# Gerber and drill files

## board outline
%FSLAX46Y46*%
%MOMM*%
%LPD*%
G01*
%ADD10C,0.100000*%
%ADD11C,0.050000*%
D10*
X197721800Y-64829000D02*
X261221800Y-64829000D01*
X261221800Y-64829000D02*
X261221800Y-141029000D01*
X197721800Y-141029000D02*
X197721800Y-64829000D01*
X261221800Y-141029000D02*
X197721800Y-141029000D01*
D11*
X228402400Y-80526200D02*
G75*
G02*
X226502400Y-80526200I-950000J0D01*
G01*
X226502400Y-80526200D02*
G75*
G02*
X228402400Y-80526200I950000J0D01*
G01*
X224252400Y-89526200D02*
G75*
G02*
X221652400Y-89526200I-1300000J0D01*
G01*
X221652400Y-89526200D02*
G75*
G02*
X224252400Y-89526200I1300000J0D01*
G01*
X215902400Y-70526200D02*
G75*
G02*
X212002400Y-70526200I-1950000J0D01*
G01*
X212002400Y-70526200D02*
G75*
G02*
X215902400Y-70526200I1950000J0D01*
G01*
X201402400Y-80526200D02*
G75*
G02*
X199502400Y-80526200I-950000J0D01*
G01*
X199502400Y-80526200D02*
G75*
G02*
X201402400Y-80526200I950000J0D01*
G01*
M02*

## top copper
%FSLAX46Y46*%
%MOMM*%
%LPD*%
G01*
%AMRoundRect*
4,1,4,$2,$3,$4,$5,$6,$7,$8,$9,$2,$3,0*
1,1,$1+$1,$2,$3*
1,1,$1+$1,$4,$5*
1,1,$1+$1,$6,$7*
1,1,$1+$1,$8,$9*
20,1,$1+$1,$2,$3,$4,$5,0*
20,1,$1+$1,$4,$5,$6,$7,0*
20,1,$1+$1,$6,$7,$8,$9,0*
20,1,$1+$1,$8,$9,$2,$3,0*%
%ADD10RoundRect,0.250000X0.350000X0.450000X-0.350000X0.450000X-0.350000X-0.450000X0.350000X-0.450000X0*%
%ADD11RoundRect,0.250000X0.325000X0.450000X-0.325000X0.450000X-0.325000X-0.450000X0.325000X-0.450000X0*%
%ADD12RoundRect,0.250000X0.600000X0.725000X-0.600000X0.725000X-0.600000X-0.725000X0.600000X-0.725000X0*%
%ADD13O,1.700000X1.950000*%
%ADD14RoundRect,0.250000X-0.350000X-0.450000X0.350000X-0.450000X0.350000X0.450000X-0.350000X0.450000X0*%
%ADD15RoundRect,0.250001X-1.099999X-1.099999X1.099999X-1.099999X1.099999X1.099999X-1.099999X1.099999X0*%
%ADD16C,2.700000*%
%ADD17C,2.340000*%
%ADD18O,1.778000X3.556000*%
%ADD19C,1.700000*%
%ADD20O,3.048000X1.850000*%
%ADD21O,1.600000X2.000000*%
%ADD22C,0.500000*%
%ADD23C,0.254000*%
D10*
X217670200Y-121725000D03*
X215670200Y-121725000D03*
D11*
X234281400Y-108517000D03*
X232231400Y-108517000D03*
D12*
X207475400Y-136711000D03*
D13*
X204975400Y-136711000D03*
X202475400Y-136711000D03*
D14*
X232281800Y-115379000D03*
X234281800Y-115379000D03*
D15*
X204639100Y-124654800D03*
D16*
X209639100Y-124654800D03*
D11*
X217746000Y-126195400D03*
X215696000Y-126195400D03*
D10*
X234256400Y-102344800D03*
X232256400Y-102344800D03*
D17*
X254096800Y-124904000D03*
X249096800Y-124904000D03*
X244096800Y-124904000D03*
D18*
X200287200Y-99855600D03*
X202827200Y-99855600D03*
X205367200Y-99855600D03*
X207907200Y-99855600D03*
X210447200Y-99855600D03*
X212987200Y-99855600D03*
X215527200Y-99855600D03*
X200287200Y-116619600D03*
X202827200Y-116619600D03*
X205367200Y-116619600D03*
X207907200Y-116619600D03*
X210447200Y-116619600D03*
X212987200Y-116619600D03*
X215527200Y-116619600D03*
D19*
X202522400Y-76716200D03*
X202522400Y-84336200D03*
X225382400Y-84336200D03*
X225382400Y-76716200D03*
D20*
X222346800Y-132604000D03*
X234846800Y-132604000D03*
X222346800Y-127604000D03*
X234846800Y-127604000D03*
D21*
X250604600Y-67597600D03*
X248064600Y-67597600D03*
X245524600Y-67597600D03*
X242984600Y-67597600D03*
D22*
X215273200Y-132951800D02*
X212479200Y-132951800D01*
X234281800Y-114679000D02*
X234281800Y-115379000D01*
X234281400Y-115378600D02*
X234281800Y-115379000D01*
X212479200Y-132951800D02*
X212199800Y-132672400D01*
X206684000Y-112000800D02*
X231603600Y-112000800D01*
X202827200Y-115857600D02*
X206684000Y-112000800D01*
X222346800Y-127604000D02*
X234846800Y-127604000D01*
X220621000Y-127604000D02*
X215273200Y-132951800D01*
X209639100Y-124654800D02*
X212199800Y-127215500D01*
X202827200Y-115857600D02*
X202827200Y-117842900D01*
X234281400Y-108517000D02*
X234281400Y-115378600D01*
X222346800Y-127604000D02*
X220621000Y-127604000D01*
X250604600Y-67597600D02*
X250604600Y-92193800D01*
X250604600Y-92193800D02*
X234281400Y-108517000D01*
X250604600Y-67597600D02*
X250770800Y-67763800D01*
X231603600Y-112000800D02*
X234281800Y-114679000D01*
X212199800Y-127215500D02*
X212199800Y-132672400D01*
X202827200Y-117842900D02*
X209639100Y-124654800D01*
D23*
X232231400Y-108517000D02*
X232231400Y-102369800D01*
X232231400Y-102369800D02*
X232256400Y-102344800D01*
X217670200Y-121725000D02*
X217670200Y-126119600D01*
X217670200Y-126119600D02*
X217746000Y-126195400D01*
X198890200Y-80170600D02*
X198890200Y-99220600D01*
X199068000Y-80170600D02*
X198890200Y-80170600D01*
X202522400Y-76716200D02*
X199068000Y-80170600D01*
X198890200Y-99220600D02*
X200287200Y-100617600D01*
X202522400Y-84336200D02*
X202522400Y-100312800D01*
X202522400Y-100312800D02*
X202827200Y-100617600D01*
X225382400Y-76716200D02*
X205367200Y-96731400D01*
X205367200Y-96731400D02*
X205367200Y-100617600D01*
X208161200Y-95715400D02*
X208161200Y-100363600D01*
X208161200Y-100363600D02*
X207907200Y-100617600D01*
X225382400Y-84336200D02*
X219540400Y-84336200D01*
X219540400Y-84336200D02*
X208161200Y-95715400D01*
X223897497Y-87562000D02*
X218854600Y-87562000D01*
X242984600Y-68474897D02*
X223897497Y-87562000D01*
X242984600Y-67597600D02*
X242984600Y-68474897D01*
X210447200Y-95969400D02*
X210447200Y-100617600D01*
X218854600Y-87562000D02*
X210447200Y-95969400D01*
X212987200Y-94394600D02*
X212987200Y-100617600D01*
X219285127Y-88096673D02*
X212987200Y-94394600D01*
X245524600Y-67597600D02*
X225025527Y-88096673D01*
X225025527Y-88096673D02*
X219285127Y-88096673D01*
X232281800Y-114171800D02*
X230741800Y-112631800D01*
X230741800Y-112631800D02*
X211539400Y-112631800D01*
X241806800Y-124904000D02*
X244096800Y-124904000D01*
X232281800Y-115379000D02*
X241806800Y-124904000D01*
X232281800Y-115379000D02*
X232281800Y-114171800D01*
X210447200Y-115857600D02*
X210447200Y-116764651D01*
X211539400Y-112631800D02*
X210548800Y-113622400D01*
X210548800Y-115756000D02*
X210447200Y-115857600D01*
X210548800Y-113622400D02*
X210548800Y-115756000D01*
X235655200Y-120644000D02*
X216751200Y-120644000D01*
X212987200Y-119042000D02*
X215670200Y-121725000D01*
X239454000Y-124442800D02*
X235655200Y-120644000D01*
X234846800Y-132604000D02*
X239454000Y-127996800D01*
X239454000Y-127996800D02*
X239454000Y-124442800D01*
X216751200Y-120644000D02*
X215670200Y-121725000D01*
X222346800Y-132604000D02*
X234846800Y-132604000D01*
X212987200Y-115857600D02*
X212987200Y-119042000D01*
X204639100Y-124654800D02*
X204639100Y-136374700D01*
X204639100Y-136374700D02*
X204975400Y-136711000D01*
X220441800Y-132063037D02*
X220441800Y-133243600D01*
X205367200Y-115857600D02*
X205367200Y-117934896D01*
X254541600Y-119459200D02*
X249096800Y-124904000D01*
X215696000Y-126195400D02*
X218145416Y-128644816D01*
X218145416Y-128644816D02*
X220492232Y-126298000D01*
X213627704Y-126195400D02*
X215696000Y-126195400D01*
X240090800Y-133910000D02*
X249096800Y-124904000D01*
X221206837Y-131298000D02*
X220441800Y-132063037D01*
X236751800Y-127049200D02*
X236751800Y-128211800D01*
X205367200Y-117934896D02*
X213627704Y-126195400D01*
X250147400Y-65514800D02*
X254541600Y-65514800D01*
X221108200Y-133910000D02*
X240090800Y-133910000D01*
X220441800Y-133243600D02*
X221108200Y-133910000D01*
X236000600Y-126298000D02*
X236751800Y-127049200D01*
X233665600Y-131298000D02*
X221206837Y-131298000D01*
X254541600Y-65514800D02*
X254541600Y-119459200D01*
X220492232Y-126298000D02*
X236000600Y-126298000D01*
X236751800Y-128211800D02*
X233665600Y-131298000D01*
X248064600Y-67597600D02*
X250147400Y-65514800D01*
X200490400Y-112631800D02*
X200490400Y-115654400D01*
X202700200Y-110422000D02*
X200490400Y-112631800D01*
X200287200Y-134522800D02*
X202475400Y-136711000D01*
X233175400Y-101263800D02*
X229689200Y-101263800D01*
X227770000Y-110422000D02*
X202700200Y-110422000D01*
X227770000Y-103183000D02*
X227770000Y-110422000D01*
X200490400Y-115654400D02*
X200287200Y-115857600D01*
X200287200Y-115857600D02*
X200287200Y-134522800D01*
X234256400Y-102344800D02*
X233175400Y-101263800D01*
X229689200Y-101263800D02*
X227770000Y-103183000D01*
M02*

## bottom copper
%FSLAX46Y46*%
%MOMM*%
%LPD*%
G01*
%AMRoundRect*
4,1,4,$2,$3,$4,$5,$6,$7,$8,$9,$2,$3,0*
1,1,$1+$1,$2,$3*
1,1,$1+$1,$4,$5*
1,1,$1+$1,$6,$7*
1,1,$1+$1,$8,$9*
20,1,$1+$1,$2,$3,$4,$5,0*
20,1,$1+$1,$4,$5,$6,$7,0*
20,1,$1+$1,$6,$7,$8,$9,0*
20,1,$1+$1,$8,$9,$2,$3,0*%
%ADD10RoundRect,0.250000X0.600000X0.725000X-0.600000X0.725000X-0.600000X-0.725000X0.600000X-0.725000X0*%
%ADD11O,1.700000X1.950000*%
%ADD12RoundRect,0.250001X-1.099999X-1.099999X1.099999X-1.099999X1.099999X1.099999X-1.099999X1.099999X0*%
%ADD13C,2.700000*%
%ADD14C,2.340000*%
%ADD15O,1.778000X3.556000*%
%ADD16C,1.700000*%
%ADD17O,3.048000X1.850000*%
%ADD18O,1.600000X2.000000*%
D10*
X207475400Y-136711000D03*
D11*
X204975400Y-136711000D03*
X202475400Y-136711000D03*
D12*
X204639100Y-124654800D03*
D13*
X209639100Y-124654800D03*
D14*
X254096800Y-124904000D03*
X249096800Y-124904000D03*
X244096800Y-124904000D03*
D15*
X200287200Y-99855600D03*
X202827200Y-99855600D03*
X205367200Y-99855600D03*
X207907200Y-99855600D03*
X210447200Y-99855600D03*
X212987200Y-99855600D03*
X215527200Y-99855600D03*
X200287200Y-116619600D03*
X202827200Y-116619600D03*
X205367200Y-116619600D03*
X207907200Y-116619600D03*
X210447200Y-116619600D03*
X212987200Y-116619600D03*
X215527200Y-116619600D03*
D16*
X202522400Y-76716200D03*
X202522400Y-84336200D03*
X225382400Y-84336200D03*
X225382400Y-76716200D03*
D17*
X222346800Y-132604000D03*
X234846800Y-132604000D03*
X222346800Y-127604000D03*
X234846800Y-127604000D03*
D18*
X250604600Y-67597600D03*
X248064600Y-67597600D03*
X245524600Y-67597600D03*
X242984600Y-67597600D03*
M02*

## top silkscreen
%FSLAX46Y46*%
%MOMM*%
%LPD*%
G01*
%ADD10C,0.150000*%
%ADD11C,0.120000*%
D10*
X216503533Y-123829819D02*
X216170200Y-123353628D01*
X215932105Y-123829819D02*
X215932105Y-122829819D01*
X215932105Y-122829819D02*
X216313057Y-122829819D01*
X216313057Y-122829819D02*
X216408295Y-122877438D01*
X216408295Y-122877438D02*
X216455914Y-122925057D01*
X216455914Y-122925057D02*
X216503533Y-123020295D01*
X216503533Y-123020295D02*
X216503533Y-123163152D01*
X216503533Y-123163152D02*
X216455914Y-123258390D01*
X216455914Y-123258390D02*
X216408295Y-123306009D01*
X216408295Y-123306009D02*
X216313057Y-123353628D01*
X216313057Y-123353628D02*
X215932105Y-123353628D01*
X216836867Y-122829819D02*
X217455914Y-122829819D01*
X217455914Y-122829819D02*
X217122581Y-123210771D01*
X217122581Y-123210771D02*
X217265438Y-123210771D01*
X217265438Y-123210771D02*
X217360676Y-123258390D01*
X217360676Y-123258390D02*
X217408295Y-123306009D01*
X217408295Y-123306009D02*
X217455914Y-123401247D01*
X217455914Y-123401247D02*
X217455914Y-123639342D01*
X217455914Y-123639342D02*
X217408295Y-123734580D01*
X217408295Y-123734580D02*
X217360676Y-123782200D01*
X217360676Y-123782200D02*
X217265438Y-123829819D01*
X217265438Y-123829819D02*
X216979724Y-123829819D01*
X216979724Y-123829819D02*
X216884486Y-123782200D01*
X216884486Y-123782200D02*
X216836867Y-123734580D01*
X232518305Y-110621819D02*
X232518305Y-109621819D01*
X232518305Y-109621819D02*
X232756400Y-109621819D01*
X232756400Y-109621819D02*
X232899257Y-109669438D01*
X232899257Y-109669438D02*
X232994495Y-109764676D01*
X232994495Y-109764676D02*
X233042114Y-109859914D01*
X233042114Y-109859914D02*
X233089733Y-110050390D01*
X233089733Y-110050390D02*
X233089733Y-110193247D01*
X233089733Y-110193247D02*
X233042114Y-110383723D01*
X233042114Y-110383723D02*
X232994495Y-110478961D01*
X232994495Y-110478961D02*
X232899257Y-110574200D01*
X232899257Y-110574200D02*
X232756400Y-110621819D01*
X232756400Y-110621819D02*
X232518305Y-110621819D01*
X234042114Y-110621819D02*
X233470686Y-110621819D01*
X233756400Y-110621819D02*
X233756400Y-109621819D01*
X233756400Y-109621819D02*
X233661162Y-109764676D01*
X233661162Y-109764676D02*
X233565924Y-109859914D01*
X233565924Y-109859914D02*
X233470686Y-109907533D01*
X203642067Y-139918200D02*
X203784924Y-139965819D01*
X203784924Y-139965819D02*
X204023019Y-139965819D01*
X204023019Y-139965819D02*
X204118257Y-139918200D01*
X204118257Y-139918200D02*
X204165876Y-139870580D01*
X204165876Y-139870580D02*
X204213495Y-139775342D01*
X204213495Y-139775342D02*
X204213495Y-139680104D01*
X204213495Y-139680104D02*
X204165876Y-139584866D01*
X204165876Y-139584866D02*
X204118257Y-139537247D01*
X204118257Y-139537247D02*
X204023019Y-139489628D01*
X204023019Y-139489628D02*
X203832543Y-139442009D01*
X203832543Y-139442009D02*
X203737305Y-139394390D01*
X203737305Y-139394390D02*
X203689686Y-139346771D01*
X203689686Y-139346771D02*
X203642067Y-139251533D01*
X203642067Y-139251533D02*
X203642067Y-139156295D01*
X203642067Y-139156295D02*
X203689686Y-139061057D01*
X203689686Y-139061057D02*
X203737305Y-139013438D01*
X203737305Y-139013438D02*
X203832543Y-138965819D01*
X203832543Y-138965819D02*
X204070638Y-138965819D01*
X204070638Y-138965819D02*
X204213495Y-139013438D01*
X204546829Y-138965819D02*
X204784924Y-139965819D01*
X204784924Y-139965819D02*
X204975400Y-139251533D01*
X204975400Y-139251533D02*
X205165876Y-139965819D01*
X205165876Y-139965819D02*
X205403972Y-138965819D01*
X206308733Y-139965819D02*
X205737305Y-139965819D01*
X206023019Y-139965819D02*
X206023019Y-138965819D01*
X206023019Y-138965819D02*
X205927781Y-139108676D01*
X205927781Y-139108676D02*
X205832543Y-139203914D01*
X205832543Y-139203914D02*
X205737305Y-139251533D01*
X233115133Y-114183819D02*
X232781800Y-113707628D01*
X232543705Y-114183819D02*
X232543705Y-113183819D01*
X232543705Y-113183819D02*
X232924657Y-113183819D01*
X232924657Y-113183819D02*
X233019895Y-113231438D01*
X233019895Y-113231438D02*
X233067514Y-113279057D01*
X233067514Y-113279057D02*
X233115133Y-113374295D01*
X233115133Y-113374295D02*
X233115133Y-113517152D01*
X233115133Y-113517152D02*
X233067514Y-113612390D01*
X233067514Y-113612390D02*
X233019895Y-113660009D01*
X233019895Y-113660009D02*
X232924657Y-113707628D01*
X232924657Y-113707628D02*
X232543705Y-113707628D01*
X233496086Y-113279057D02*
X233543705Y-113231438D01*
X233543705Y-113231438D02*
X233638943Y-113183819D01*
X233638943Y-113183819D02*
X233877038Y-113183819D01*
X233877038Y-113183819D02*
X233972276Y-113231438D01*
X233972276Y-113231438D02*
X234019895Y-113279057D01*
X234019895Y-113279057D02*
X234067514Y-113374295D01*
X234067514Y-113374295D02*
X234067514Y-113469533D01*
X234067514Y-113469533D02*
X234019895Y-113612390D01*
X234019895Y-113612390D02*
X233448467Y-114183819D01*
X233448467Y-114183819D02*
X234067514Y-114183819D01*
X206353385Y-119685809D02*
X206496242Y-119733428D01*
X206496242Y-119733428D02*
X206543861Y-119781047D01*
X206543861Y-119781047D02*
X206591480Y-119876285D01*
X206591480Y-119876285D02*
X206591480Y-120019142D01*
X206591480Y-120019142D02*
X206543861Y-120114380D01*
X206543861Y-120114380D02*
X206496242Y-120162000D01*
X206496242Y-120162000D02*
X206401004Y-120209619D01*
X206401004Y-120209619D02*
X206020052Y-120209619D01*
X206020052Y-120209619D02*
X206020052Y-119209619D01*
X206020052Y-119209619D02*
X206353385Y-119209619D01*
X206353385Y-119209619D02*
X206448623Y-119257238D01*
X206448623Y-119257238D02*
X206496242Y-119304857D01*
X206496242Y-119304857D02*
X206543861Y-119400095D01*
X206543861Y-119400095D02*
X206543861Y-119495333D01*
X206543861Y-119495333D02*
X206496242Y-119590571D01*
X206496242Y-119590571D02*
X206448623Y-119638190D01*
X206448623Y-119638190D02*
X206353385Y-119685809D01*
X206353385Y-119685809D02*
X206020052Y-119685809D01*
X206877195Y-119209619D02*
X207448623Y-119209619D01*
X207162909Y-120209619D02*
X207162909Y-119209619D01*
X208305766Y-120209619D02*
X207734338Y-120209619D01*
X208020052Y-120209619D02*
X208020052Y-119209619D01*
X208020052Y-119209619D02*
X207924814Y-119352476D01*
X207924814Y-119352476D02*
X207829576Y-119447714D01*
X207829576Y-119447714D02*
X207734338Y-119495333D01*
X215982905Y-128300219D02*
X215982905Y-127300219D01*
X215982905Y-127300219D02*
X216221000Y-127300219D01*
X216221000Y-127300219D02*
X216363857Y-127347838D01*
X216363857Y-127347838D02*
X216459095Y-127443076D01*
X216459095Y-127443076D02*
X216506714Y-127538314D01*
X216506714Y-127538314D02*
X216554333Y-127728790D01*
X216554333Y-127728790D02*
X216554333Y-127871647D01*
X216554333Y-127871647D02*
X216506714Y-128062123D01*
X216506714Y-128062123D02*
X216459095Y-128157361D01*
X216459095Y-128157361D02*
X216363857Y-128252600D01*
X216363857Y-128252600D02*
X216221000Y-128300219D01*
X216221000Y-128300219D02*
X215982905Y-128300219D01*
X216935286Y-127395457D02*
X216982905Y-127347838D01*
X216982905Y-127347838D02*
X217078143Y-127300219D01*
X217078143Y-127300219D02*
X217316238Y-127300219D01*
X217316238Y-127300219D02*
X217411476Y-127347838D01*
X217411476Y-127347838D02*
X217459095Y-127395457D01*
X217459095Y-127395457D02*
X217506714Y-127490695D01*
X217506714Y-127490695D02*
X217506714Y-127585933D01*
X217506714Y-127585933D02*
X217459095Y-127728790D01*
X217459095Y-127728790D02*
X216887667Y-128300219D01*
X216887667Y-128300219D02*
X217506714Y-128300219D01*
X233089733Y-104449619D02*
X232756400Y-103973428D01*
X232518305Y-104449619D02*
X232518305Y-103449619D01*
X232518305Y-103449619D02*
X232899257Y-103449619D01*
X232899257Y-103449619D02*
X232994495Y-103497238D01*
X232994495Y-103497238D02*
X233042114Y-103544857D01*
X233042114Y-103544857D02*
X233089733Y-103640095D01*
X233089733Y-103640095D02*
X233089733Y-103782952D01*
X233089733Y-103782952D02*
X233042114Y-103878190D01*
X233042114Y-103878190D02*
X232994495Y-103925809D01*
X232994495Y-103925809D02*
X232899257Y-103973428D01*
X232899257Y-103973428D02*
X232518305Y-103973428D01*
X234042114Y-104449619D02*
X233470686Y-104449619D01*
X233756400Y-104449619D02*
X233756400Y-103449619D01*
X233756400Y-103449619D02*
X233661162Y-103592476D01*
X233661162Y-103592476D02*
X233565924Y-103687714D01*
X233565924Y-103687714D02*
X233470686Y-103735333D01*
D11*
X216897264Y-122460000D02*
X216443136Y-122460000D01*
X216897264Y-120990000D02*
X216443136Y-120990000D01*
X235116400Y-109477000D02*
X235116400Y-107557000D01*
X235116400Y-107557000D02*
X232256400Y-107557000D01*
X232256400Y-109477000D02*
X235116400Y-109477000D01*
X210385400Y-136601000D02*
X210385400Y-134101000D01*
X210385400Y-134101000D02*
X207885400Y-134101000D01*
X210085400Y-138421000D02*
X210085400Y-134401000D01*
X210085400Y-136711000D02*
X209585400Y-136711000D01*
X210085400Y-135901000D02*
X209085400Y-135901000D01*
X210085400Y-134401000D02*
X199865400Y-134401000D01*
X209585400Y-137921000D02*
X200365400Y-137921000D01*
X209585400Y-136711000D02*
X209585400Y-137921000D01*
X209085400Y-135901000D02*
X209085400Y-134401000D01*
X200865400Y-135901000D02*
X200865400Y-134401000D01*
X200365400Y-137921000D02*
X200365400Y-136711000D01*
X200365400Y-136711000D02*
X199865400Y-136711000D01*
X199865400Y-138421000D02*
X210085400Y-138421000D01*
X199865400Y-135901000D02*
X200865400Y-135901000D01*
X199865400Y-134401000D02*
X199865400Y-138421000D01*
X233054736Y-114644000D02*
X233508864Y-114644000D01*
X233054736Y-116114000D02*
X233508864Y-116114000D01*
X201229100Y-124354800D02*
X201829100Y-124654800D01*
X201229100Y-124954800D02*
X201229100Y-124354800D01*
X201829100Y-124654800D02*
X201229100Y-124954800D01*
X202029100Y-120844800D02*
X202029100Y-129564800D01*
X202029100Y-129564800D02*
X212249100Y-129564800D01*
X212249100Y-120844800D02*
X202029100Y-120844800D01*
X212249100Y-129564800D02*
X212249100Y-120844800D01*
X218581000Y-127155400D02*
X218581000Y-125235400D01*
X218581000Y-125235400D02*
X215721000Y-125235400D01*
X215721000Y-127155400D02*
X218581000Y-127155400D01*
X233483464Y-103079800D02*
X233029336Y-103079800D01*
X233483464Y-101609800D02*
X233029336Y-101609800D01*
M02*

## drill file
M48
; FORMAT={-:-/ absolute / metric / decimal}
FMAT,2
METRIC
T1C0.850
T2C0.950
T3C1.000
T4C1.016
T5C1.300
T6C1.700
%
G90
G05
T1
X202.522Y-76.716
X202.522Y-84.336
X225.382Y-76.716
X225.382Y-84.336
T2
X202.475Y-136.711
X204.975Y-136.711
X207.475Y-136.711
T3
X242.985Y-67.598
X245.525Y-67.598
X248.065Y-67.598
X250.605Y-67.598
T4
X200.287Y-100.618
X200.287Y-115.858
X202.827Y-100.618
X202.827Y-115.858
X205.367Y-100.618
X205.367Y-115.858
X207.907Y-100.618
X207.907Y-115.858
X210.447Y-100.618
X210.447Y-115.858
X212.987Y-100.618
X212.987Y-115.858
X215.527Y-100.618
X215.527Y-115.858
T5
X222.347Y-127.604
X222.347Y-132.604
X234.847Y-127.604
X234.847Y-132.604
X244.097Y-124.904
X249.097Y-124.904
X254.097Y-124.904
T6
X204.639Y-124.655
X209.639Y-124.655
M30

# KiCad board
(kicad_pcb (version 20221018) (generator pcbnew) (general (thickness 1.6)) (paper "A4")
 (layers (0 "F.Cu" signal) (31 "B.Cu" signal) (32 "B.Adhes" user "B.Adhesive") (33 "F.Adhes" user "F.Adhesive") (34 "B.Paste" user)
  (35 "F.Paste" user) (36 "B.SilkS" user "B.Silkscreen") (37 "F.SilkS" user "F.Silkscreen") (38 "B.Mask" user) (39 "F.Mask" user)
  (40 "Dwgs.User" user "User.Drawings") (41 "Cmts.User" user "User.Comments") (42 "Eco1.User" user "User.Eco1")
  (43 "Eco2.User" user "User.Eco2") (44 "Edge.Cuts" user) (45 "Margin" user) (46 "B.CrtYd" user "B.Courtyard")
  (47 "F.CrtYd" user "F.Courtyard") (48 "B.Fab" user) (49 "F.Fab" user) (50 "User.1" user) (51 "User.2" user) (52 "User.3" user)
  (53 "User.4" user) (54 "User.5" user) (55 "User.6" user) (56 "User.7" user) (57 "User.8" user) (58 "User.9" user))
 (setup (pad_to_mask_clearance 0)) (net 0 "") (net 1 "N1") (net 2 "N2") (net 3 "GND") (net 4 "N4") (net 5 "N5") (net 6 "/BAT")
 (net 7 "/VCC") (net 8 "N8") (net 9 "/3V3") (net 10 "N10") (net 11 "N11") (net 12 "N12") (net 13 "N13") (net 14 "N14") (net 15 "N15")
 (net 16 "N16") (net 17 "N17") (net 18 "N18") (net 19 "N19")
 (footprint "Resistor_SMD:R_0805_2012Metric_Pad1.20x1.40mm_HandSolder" (layer "F.Cu") (at 216.6702 121.725 180)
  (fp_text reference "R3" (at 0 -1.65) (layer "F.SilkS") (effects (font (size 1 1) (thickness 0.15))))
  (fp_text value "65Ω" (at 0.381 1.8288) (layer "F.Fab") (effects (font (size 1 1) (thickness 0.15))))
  (fp_line (start -0.227064 -0.735) (end 0.227064 -0.735) (stroke (width 0.12) (type solid)) (layer "F.SilkS"))
  (fp_line (start -0.227064 0.735) (end 0.227064 0.735) (stroke (width 0.12) (type solid)) (layer "F.SilkS"))
  (pad "1" smd roundrect (at -1 0 180) (size 1.2 1.4) (layers "F.Cu" "F.Paste" "F.Mask") (roundrect_rratio 0.2083333333) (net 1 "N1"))
  (pad "2" smd roundrect (at 1 0 180) (size 1.2 1.4) (layers "F.Cu" "F.Paste" "F.Mask") (roundrect_rratio 0.2083333333) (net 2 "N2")))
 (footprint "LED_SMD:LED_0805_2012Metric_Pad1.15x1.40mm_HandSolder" (layer "F.Cu") (at 233.2564 108.517 180)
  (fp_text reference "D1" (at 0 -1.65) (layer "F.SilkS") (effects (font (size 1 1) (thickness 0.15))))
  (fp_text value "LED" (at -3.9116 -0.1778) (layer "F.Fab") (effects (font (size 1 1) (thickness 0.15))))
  (fp_line (start -1.86 -0.96) (end -1.86 0.96) (stroke (width 0.12) (type solid)) (layer "F.SilkS"))
  (fp_line (start -1.86 0.96) (end 1 0.96) (stroke (width 0.12) (type solid)) (layer "F.SilkS"))
  (fp_line (start 1 -0.96) (end -1.86 -0.96) (stroke (width 0.12) (type solid)) (layer "F.SilkS"))
  (pad "1" smd roundrect (at -1.025 0 180) (size 1.15 1.4) (layers "F.Cu" "F.Paste" "F.Mask") (roundrect_rratio 0.2173913043) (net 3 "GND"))
  (pad "2" smd roundrect (at 1.025 0 180) (size 1.15 1.4) (layers "F.Cu" "F.Paste" "F.Mask") (roundrect_rratio 0.2173913043) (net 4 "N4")))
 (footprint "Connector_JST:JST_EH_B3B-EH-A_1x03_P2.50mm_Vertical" (layer "F.Cu") (at 207.4754 136.711 180)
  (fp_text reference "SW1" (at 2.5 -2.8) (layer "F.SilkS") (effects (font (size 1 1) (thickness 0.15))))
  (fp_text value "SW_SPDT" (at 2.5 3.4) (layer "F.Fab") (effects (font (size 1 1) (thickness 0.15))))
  (fp_line (start -2.91 0.11) (end -2.91 2.61) (stroke (width 0.12) (type solid)) (layer "F.SilkS"))
  (fp_line (start -2.91 2.61) (end -0.41 2.61) (stroke (width 0.12) (type solid)) (layer "F.SilkS"))
  (fp_line (start -2.61 -1.71) (end -2.61 2.31) (stroke (width 0.12) (type solid)) (layer "F.SilkS"))
  (fp_line (start -2.61 0) (end -2.11 0) (stroke (width 0.12) (type solid)) (layer "F.SilkS"))
  (fp_line (start -2.61 0.81) (end -1.61 0.81) (stroke (width 0.12) (type solid)) (layer "F.SilkS"))
  (fp_line (start -2.61 2.31) (end 7.61 2.31) (stroke (width 0.12) (type solid)) (layer "F.SilkS"))
  (fp_line (start -2.11 -1.21) (end 7.11 -1.21) (stroke (width 0.12) (type solid)) (layer "F.SilkS"))
  (fp_line (start -2.11 0) (end -2.11 -1.21) (stroke (width 0.12) (type solid)) (layer "F.SilkS"))
  (fp_line (start -1.61 0.81) (end -1.61 2.31) (stroke (width 0.12) (type solid)) (layer "F.SilkS"))
  (fp_line (start 6.61 0.81) (end 6.61 2.31) (stroke (width 0.12) (type solid)) (layer "F.SilkS"))
  (fp_line (start 7.11 -1.21) (end 7.11 0) (stroke (width 0.12) (type solid)) (layer "F.SilkS"))
  (fp_line (start 7.11 0) (end 7.61 0) (stroke (width 0.12) (type solid)) (layer "F.SilkS"))
  (fp_line (start 7.61 -1.71) (end -2.61 -1.71) (stroke (width 0.12) (type solid)) (layer "F.SilkS"))
  (fp_line (start 7.61 0.81) (end 6.61 0.81) (stroke (width 0.12) (type solid)) (layer "F.SilkS"))
  (fp_line (start 7.61 2.31) (end 7.61 -1.71) (stroke (width 0.12) (type solid)) (layer "F.SilkS"))
  (pad "1" thru_hole roundrect (at 0 0 180) (size 1.7 1.95) (drill 0.95) (layers "*.Cu" "*.Mask") (roundrect_rratio 0.1470588235)
   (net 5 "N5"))
  (pad "2" thru_hole oval (at 2.5 0 180) (size 1.7 1.95) (drill 0.95) (layers "*.Cu" "*.Mask") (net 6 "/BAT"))
  (pad "3" thru_hole oval (at 5 0 180) (size 1.7 1.95) (drill 0.95) (layers "*.Cu" "*.Mask") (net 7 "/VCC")))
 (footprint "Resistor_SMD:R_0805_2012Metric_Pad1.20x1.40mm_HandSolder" (layer "F.Cu") (at 233.2818 115.379)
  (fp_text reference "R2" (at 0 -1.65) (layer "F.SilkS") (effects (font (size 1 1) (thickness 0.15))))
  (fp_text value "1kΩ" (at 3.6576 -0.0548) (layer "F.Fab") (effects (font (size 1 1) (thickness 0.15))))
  (fp_line (start -0.227064 -0.735) (end 0.227064 -0.735) (stroke (width 0.12) (type solid)) (layer "F.SilkS"))
  (fp_line (start -0.227064 0.735) (end 0.227064 0.735) (stroke (width 0.12) (type solid)) (layer "F.SilkS"))
  (pad "1" smd roundrect (at -1 0) (size 1.2 1.4) (layers "F.Cu" "F.Paste" "F.Mask") (roundrect_rratio 0.2083333333) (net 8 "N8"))
  (pad "2" smd roundrect (at 1 0) (size 1.2 1.4) (layers "F.Cu" "F.Paste" "F.Mask") (roundrect_rratio 0.2083333333) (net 3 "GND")))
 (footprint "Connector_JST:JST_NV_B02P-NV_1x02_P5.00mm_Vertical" (layer "F.Cu") (at 204.6391 124.6548)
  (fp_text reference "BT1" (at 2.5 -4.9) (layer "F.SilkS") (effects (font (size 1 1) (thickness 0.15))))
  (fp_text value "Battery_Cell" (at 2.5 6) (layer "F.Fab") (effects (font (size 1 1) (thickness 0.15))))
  (fp_line (start -3.41 -0.3) (end -2.81 0) (stroke (width 0.12) (type solid)) (layer "F.SilkS"))
  (fp_line (start -3.41 0.3) (end -3.41 -0.3) (stroke (width 0.12) (type solid)) (layer "F.SilkS"))
  (fp_line (start -2.81 0) (end -3.41 0.3) (stroke (width 0.12) (type solid)) (layer "F.SilkS"))
  (fp_line (start -2.61 -3.81) (end -2.61 4.91) (stroke (width 0.12) (type solid)) (layer "F.SilkS"))
  (fp_line (start -2.61 4.91) (end 7.61 4.91) (stroke (width 0.12) (type solid)) (layer "F.SilkS"))
  (fp_line (start 7.61 -3.81) (end -2.61 -3.81) (stroke (width 0.12) (type solid)) (layer "F.SilkS"))
  (fp_line (start 7.61 4.91) (end 7.61 -3.81) (stroke (width 0.12) (type solid)) (layer "F.SilkS"))
  (pad "1" thru_hole roundrect (at 0 0) (size 2.7 2.7) (drill 1.7) (layers "*.Cu" "*.Mask") (roundrect_rratio 0.09259296296) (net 6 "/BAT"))
  (pad "2" thru_hole circle (at 5 0) (size 2.7 2.7) (drill 1.7) (layers "*.Cu" "*.Mask") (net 3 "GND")))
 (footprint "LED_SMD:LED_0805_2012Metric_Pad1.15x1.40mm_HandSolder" (layer "F.Cu") (at 216.721 126.1954 180)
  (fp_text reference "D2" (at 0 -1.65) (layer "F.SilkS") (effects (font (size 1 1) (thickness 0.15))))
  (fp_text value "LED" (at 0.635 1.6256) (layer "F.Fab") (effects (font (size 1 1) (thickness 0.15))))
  (fp_line (start -1.86 -0.96) (end -1.86 0.96) (stroke (width 0.12) (type solid)) (layer "F.SilkS"))
  (fp_line (start -1.86 0.96) (end 1 0.96) (stroke (width 0.12) (type solid)) (layer "F.SilkS"))
  (fp_line (start 1 -0.96) (end -1.86 -0.96) (stroke (width 0.12) (type solid)) (layer "F.SilkS"))
  (pad "1" smd roundrect (at -1.025 0 180) (size 1.15 1.4) (layers "F.Cu" "F.Paste" "F.Mask") (roundrect_rratio 0.2173913043) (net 1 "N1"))
  (pad "2" smd roundrect (at 1.025 0 180) (size 1.15 1.4) (layers "F.Cu" "F.Paste" "F.Mask") (roundrect_rratio 0.2173913043) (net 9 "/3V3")))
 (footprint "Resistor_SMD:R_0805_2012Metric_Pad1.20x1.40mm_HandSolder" (layer "F.Cu") (at 233.2564 102.3448 180)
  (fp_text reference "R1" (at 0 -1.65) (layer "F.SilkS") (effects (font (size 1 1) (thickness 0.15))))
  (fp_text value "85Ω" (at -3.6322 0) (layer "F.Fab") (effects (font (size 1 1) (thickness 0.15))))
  (fp_line (start -0.227064 -0.735) (end 0.227064 -0.735) (stroke (width 0.12) (type solid)) (layer "F.SilkS"))
  (fp_line (start -0.227064 0.735) (end 0.227064 0.735) (stroke (width 0.12) (type solid)) (layer "F.SilkS"))
  (pad "1" smd roundrect (at -1 0 180) (size 1.2 1.4) (layers "F.Cu" "F.Paste" "F.Mask") (roundrect_rratio 0.2083333333) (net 7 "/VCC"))
  (pad "2" smd roundrect (at 1 0 180) (size 1.2 1.4) (layers "F.Cu" "F.Paste" "F.Mask") (roundrect_rratio 0.2083333333) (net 4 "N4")))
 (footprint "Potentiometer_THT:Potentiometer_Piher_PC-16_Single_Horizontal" (layer "B.Cu") (at 254.0968 124.904 -90)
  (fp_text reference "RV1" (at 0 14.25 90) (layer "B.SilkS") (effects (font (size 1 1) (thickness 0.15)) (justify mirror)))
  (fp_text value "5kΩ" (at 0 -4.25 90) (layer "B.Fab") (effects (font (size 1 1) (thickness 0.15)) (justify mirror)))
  (pad "1" thru_hole circle (at 0 0 270) (size 2.34 2.34) (drill 1.3) (layers "*.Cu" "*.Mask") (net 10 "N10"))
  (pad "2" thru_hole circle (at 0 5 270) (size 2.34 2.34) (drill 1.3) (layers "*.Cu" "*.Mask") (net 9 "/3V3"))
  (pad "3" thru_hole circle (at 0 10 270) (size 2.34 2.34) (drill 1.3) (layers "*.Cu" "*.Mask") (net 8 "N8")))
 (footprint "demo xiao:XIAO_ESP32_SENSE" (layer "B.Cu") (at 207.9072 108.2376 -90)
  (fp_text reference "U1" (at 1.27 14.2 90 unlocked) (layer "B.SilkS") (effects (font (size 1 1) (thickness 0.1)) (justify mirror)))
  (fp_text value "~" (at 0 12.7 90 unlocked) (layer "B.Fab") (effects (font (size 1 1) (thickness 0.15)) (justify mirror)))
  (pad "1" thru_hole oval (at -7.62 7.62 270) (size 3.556 1.778) (drill 1.016 (offset -0.762 0)) (layers "*.Cu" "*.Mask") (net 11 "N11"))
  (pad "2" thru_hole oval (at -7.62 5.08 270) (size 3.556 1.778) (drill 1.016 (offset -0.762 0)) (layers "*.Cu" "*.Mask") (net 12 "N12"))
  (pad "3" thru_hole oval (at -7.62 2.54 270) (size 3.556 1.778) (drill 1.016 (offset -0.762 0)) (layers "*.Cu" "*.Mask") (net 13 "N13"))
  (pad "4" thru_hole oval (at -7.62 0 270) (size 3.556 1.778) (drill 1.016 (offset -0.762 0)) (layers "*.Cu" "*.Mask") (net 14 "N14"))
  (pad "5" thru_hole oval (at -7.62 -2.54 270) (size 3.556 1.778) (drill 1.016 (offset -0.762 0)) (layers "*.Cu" "*.Mask") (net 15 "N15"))
  (pad "6" thru_hole oval (at -7.62 -5.08 270) (size 3.556 1.778) (drill 1.016 (offset -0.762 0)) (layers "*.Cu" "*.Mask") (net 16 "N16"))
  (pad "7" thru_hole oval (at -7.62 -7.62 270) (size 3.556 1.778) (drill 1.016 (offset -0.762 0)) (layers "*.Cu" "*.Mask") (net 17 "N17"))
  (pad "8" thru_hole oval (at 7.62 7.62 270) (size 3.556 1.778) (drill 1.016 (offset 0.762 0)) (layers "*.Cu" "*.Mask") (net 7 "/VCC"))
  (pad "9" thru_hole oval (at 7.62 5.08 270) (size 3.556 1.778) (drill 1.016 (offset 0.762 0)) (layers "*.Cu" "*.Mask") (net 3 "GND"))
  (pad "10" thru_hole oval (at 7.62 2.54 270) (size 3.556 1.778) (drill 1.016 (offset 0.762 0)) (layers "*.Cu" "*.Mask") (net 9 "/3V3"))
  (pad "11" thru_hole oval (at 7.62 0 270) (size 3.556 1.778) (drill 1.016 (offset 0.762 0)) (layers "*.Cu" "*.Mask") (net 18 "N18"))
  (pad "12" thru_hole oval (at 7.62 -2.54 270) (size 3.556 1.778) (drill 1.016 (offset 0.762 0)) (layers "*.Cu" "*.Mask") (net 8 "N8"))
  (pad "13" thru_hole oval (at 7.62 -5.08 270) (size 3.556 1.778) (drill 1.016 (offset 0.762 0)) (layers "*.Cu" "*.Mask") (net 2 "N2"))
  (pad "14" thru_hole oval (at 7.62 -7.62 270) (size 3.556 1.778) (drill 1.016 (offset 0.762 0)) (layers "*.Cu" "*.Mask") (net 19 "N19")))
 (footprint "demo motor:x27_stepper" (layer "B.Cu") (at 211.4124 90.6862 180)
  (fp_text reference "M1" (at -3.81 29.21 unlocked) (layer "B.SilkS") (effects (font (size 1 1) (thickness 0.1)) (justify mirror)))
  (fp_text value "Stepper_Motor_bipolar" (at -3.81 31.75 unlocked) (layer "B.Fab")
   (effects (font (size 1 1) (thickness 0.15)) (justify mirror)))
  (fp_circle (center -16.04 10.16) (end -15.09 10.16) (stroke (width 0.05) (type default)) (fill none) (layer "Edge.Cuts"))
  (fp_circle (center -11.54 1.16) (end -10.24 1.16) (stroke (width 0.05) (type default)) (fill none) (layer "Edge.Cuts"))
  (fp_circle (center -2.54 20.16) (end -0.59 20.16) (stroke (width 0.05) (type default)) (fill none) (layer "Edge.Cuts"))
  (fp_circle (center 10.96 10.16) (end 11.91 10.16) (stroke (width 0.05) (type default)) (fill none) (layer "Edge.Cuts"))
  (pad "1" thru_hole circle (at 8.89 13.97 180) (size 1.7 1.7) (drill 0.85) (layers "*.Cu" "*.Mask") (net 11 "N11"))
  (pad "2" thru_hole circle (at 8.89 6.35 180) (size 1.7 1.7) (drill 0.85) (layers "*.Cu" "*.Mask") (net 12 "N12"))
  (pad "3" thru_hole circle (at -13.97 6.35 180) (size 1.7 1.7) (drill 0.85) (layers "*.Cu" "*.Mask") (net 14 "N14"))
  (pad "4" thru_hole circle (at -13.97 13.97 180) (size 1.7 1.7) (drill 0.85) (layers "*.Cu" "*.Mask") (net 13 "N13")))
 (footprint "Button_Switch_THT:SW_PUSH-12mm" (layer "B.Cu") (at 222.3468 132.604)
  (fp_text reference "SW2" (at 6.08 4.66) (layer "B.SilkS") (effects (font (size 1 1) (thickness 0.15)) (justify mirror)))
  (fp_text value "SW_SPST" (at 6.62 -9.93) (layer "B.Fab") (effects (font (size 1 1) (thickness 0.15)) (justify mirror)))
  (pad "1" thru_hole oval (at 0 0) (size 3.048 1.85) (drill 1.3) (layers "*.Cu" "*.Mask") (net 2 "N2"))
  (pad "1" thru_hole oval (at 12.5 0) (size 3.048 1.85) (drill 1.3) (layers "*.Cu" "*.Mask") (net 2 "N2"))
  (pad "2" thru_hole oval (at 0 -5) (size 3.048 1.85) (drill 1.3) (layers "*.Cu" "*.Mask") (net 3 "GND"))
  (pad "2" thru_hole oval (at 12.5 -5) (size 3.048 1.85) (drill 1.3) (layers "*.Cu" "*.Mask") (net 3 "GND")))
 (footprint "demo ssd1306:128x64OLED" (layer "B.Cu") (at 246.9846 78.1976 180)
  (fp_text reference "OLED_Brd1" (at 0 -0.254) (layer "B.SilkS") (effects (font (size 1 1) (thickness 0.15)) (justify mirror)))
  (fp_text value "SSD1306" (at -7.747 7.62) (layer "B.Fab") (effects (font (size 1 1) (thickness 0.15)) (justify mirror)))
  (pad "1" thru_hole oval (at -3.62 10.6 90) (size 2 1.6) (drill 1) (layers "*.Cu" "*.Mask") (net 3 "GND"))
  (pad "2" thru_hole oval (at -1.08 10.6 90) (size 2 1.6) (drill 1) (layers "*.Cu" "*.Mask") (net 9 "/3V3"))
  (pad "3" thru_hole oval (at 1.46 10.6 90) (size 2 1.6) (drill 1) (layers "*.Cu" "*.Mask") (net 16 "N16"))
  (pad "4" thru_hole oval (at 4 10.6 90) (size 2 1.6) (drill 1) (layers "*.Cu" "*.Mask") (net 15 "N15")))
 (gr_line (start 197.7218 64.829) (end 261.2218 64.829) (stroke (width 0.1) (type default)) (layer "Edge.Cuts"))
 (gr_line (start 261.2218 64.829) (end 261.2218 141.029) (stroke (width 0.1) (type default)) (layer "Edge.Cuts"))
 (gr_line (start 197.7218 141.029) (end 197.7218 64.829) (stroke (width 0.1) (type default)) (layer "Edge.Cuts"))
 (gr_line (start 261.2218 141.029) (end 197.7218 141.029) (stroke (width 0.1) (type default)) (layer "Edge.Cuts"))
 (segment (start 215.2732 132.9518) (end 212.4792 132.9518) (width 0.5) (layer "F.Cu") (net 3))
 (segment (start 234.2818 114.679) (end 234.2818 115.379) (width 0.5) (layer "F.Cu") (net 3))
 (segment (start 234.2814 115.3786) (end 234.2818 115.379) (width 0.5) (layer "F.Cu") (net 3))
 (segment (start 212.4792 132.9518) (end 212.1998 132.6724) (width 0.5) (layer "F.Cu") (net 3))
 (segment (start 206.684 112.0008) (end 231.6036 112.0008) (width 0.5) (layer "F.Cu") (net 3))
 (segment (start 202.8272 115.8576) (end 206.684 112.0008) (width 0.5) (layer "F.Cu") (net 3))
 (segment (start 222.3468 127.604) (end 234.8468 127.604) (width 0.5) (layer "F.Cu") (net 3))
 (segment (start 220.621 127.604) (end 215.2732 132.9518) (width 0.5) (layer "F.Cu") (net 3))
 (segment (start 209.6391 124.6548) (end 212.1998 127.2155) (width 0.5) (layer "F.Cu") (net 3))
 (segment (start 202.8272 115.8576) (end 202.8272 117.8429) (width 0.5) (layer "F.Cu") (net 3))
 (segment (start 234.2814 108.517) (end 234.2814 115.3786) (width 0.5) (layer "F.Cu") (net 3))
 (segment (start 222.3468 127.604) (end 220.621 127.604) (width 0.5) (layer "F.Cu") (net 3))
 (segment (start 250.6046 67.5976) (end 250.6046 92.1938) (width 0.5) (layer "F.Cu") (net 3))
 (segment (start 250.6046 92.1938) (end 234.2814 108.517) (width 0.5) (layer "F.Cu") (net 3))
 (segment (start 250.6046 67.5976) (end 250.7708 67.7638) (width 0.5) (layer "F.Cu") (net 3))
 (segment (start 231.6036 112.0008) (end 234.2818 114.679) (width 0.5) (layer "F.Cu") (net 3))
 (segment (start 212.1998 127.2155) (end 212.1998 132.6724) (width 0.5) (layer "F.Cu") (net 3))
 (segment (start 202.8272 117.8429) (end 209.6391 124.6548) (width 0.5) (layer "F.Cu") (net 3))
 (segment (start 232.2314 108.517) (end 232.2314 102.3698) (width 0.254) (layer "F.Cu") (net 4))
 (segment (start 232.2314 102.3698) (end 232.2564 102.3448) (width 0.254) (layer "F.Cu") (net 4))
 (segment (start 217.6702 121.725) (end 217.6702 126.1196) (width 0.254) (layer "F.Cu") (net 1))
 (segment (start 217.6702 126.1196) (end 217.746 126.1954) (width 0.254) (layer "F.Cu") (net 1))
 (segment (start 198.8902 80.1706) (end 198.8902 99.2206) (width 0.254) (layer "F.Cu") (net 11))
 (segment (start 199.068 80.1706) (end 198.8902 80.1706) (width 0.254) (layer "F.Cu") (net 11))
 (segment (start 202.5224 76.7162) (end 199.068 80.1706) (width 0.254) (layer "F.Cu") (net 11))
 (segment (start 198.8902 99.2206) (end 200.2872 100.6176) (width 0.254) (layer "F.Cu") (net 11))
 (segment (start 202.5224 84.3362) (end 202.5224 100.3128) (width 0.254) (layer "F.Cu") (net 12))
 (segment (start 202.5224 100.3128) (end 202.8272 100.6176) (width 0.254) (layer "F.Cu") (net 12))
 (segment (start 225.3824 76.7162) (end 205.3672 96.7314) (width 0.254) (layer "F.Cu") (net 13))
 (segment (start 205.3672 96.7314) (end 205.3672 100.6176) (width 0.254) (layer "F.Cu") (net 13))
 (segment (start 208.1612 95.7154) (end 208.1612 100.3636) (width 0.254) (layer "F.Cu") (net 14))
 (segment (start 208.1612 100.3636) (end 207.9072 100.6176) (width 0.254) (layer "F.Cu") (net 14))
 (segment (start 225.3824 84.3362) (end 219.5404 84.3362) (width 0.254) (layer "F.Cu") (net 14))
 (segment (start 219.5404 84.3362) (end 208.1612 95.7154) (width 0.254) (layer "F.Cu") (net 14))
 (segment (start 223.897497 87.562) (end 218.8546 87.562) (width 0.254) (layer "F.Cu") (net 15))
 (segment (start 242.9846 68.474897) (end 223.897497 87.562) (width 0.254) (layer "F.Cu") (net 15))
 (segment (start 242.9846 67.5976) (end 242.9846 68.474897) (width 0.254) (layer "F.Cu") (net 15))
 (segment (start 210.4472 95.9694) (end 210.4472 100.6176) (width 0.254) (layer "F.Cu") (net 15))
 (segment (start 218.8546 87.562) (end 210.4472 95.9694) (width 0.254) (layer "F.Cu") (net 15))
 (segment (start 212.9872 94.3946) (end 212.9872 100.6176) (width 0.254) (layer "F.Cu") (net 16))
 (segment (start 219.285127 88.096673) (end 212.9872 94.3946) (width 0.254) (layer "F.Cu") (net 16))
 (segment (start 245.5246 67.5976) (end 225.025527 88.096673) (width 0.254) (layer "F.Cu") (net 16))
 (segment (start 225.025527 88.096673) (end 219.285127 88.096673) (width 0.254) (layer "F.Cu") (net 16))
 (segment (start 232.2818 114.1718) (end 230.7418 112.6318) (width 0.254) (layer "F.Cu") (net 8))
 (segment (start 230.7418 112.6318) (end 211.5394 112.6318) (width 0.254) (layer "F.Cu") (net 8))
 (segment (start 241.8068 124.904) (end 244.0968 124.904) (width 0.254) (layer "F.Cu") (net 8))
 (segment (start 232.2818 115.379) (end 241.8068 124.904) (width 0.254) (layer "F.Cu") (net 8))
 (segment (start 232.2818 115.379) (end 232.2818 114.1718) (width 0.254) (layer "F.Cu") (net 8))
 (segment (start 210.4472 115.8576) (end 210.4472 116.764651) (width 0.254) (layer "F.Cu") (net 8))
 (segment (start 211.5394 112.6318) (end 210.5488 113.6224) (width 0.254) (layer "F.Cu") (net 8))
 (segment (start 210.5488 115.756) (end 210.4472 115.8576) (width 0.254) (layer "F.Cu") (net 8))
 (segment (start 210.5488 113.6224) (end 210.5488 115.756) (width 0.254) (layer "F.Cu") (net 8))
 (segment (start 235.6552 120.644) (end 216.7512 120.644) (width 0.254) (layer "F.Cu") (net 2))
 (segment (start 212.9872 119.042) (end 215.6702 121.725) (width 0.254) (layer "F.Cu") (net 2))
 (segment (start 239.454 124.4428) (end 235.6552 120.644) (width 0.254) (layer "F.Cu") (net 2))
 (segment (start 234.8468 132.604) (end 239.454 127.9968) (width 0.254) (layer "F.Cu") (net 2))
 (segment (start 239.454 127.9968) (end 239.454 124.4428) (width 0.254) (layer "F.Cu") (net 2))
 (segment (start 216.7512 120.644) (end 215.6702 121.725) (width 0.254) (layer "F.Cu") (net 2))
 (segment (start 222.3468 132.604) (end 234.8468 132.604) (width 0.254) (layer "F.Cu") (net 2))
 (segment (start 212.9872 115.8576) (end 212.9872 119.042) (width 0.254) (layer "F.Cu") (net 2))
 (segment (start 204.6391 124.6548) (end 204.6391 136.3747) (width 0.254) (layer "F.Cu") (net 6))
 (segment (start 204.6391 136.3747) (end 204.9754 136.711) (width 0.254) (layer "F.Cu") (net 6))
 (segment (start 220.4418 132.063037) (end 220.4418 133.2436) (width 0.254) (layer "F.Cu") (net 9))
 (segment (start 205.3672 115.8576) (end 205.3672 117.934896) (width 0.254) (layer "F.Cu") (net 9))
 (segment (start 254.5416 119.4592) (end 249.0968 124.904) (width 0.254) (layer "F.Cu") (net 9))
 (segment (start 215.696 126.1954) (end 218.145416 128.644816) (width 0.254) (layer "F.Cu") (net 9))
 (segment (start 218.145416 128.644816) (end 220.492232 126.298) (width 0.254) (layer "F.Cu") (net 9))
 (segment (start 213.627704 126.1954) (end 215.696 126.1954) (width 0.254) (layer "F.Cu") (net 9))
 (segment (start 240.0908 133.91) (end 249.0968 124.904) (width 0.254) (layer "F.Cu") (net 9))
 (segment (start 221.206837 131.298) (end 220.4418 132.063037) (width 0.254) (layer "F.Cu") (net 9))
 (segment (start 236.7518 127.0492) (end 236.7518 128.2118) (width 0.254) (layer "F.Cu") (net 9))
 (segment (start 205.3672 117.934896) (end 213.627704 126.1954) (width 0.254) (layer "F.Cu") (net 9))
 (segment (start 250.1474 65.5148) (end 254.5416 65.5148) (width 0.254) (layer "F.Cu") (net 9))
 (segment (start 221.1082 133.91) (end 240.0908 133.91) (width 0.254) (layer "F.Cu") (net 9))
 (segment (start 220.4418 133.2436) (end 221.1082 133.91) (width 0.254) (layer "F.Cu") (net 9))
 (segment (start 236.0006 126.298) (end 236.7518 127.0492) (width 0.254) (layer "F.Cu") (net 9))
 (segment (start 233.6656 131.298) (end 221.206837 131.298) (width 0.254) (layer "F.Cu") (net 9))
 (segment (start 254.5416 65.5148) (end 254.5416 119.4592) (width 0.254) (layer "F.Cu") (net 9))
 (segment (start 220.492232 126.298) (end 236.0006 126.298) (width 0.254) (layer "F.Cu") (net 9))
 (segment (start 236.7518 128.2118) (end 233.6656 131.298) (width 0.254) (layer "F.Cu") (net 9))
 (segment (start 248.0646 67.5976) (end 250.1474 65.5148) (width 0.254) (layer "F.Cu") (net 9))
 (segment (start 200.4904 112.6318) (end 200.4904 115.6544) (width 0.254) (layer "F.Cu") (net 7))
 (segment (start 202.7002 110.422) (end 200.4904 112.6318) (width 0.254) (layer "F.Cu") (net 7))
 (segment (start 200.2872 134.5228) (end 202.4754 136.711) (width 0.254) (layer "F.Cu") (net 7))
 (segment (start 233.1754 101.2638) (end 229.6892 101.2638) (width 0.254) (layer "F.Cu") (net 7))
 (segment (start 227.77 110.422) (end 202.7002 110.422) (width 0.254) (layer "F.Cu") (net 7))
 (segment (start 227.77 103.183) (end 227.77 110.422) (width 0.254) (layer "F.Cu") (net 7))
 (segment (start 200.4904 115.6544) (end 200.2872 115.8576) (width 0.254) (layer "F.Cu") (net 7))
 (segment (start 200.2872 115.8576) (end 200.2872 134.5228) (width 0.254) (layer "F.Cu") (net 7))
 (segment (start 234.2564 102.3448) (end 233.1754 101.2638) (width 0.254) (layer "F.Cu") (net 7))
 (segment (start 229.6892 101.2638) (end 227.77 103.183) (width 0.254) (layer "F.Cu") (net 7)))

